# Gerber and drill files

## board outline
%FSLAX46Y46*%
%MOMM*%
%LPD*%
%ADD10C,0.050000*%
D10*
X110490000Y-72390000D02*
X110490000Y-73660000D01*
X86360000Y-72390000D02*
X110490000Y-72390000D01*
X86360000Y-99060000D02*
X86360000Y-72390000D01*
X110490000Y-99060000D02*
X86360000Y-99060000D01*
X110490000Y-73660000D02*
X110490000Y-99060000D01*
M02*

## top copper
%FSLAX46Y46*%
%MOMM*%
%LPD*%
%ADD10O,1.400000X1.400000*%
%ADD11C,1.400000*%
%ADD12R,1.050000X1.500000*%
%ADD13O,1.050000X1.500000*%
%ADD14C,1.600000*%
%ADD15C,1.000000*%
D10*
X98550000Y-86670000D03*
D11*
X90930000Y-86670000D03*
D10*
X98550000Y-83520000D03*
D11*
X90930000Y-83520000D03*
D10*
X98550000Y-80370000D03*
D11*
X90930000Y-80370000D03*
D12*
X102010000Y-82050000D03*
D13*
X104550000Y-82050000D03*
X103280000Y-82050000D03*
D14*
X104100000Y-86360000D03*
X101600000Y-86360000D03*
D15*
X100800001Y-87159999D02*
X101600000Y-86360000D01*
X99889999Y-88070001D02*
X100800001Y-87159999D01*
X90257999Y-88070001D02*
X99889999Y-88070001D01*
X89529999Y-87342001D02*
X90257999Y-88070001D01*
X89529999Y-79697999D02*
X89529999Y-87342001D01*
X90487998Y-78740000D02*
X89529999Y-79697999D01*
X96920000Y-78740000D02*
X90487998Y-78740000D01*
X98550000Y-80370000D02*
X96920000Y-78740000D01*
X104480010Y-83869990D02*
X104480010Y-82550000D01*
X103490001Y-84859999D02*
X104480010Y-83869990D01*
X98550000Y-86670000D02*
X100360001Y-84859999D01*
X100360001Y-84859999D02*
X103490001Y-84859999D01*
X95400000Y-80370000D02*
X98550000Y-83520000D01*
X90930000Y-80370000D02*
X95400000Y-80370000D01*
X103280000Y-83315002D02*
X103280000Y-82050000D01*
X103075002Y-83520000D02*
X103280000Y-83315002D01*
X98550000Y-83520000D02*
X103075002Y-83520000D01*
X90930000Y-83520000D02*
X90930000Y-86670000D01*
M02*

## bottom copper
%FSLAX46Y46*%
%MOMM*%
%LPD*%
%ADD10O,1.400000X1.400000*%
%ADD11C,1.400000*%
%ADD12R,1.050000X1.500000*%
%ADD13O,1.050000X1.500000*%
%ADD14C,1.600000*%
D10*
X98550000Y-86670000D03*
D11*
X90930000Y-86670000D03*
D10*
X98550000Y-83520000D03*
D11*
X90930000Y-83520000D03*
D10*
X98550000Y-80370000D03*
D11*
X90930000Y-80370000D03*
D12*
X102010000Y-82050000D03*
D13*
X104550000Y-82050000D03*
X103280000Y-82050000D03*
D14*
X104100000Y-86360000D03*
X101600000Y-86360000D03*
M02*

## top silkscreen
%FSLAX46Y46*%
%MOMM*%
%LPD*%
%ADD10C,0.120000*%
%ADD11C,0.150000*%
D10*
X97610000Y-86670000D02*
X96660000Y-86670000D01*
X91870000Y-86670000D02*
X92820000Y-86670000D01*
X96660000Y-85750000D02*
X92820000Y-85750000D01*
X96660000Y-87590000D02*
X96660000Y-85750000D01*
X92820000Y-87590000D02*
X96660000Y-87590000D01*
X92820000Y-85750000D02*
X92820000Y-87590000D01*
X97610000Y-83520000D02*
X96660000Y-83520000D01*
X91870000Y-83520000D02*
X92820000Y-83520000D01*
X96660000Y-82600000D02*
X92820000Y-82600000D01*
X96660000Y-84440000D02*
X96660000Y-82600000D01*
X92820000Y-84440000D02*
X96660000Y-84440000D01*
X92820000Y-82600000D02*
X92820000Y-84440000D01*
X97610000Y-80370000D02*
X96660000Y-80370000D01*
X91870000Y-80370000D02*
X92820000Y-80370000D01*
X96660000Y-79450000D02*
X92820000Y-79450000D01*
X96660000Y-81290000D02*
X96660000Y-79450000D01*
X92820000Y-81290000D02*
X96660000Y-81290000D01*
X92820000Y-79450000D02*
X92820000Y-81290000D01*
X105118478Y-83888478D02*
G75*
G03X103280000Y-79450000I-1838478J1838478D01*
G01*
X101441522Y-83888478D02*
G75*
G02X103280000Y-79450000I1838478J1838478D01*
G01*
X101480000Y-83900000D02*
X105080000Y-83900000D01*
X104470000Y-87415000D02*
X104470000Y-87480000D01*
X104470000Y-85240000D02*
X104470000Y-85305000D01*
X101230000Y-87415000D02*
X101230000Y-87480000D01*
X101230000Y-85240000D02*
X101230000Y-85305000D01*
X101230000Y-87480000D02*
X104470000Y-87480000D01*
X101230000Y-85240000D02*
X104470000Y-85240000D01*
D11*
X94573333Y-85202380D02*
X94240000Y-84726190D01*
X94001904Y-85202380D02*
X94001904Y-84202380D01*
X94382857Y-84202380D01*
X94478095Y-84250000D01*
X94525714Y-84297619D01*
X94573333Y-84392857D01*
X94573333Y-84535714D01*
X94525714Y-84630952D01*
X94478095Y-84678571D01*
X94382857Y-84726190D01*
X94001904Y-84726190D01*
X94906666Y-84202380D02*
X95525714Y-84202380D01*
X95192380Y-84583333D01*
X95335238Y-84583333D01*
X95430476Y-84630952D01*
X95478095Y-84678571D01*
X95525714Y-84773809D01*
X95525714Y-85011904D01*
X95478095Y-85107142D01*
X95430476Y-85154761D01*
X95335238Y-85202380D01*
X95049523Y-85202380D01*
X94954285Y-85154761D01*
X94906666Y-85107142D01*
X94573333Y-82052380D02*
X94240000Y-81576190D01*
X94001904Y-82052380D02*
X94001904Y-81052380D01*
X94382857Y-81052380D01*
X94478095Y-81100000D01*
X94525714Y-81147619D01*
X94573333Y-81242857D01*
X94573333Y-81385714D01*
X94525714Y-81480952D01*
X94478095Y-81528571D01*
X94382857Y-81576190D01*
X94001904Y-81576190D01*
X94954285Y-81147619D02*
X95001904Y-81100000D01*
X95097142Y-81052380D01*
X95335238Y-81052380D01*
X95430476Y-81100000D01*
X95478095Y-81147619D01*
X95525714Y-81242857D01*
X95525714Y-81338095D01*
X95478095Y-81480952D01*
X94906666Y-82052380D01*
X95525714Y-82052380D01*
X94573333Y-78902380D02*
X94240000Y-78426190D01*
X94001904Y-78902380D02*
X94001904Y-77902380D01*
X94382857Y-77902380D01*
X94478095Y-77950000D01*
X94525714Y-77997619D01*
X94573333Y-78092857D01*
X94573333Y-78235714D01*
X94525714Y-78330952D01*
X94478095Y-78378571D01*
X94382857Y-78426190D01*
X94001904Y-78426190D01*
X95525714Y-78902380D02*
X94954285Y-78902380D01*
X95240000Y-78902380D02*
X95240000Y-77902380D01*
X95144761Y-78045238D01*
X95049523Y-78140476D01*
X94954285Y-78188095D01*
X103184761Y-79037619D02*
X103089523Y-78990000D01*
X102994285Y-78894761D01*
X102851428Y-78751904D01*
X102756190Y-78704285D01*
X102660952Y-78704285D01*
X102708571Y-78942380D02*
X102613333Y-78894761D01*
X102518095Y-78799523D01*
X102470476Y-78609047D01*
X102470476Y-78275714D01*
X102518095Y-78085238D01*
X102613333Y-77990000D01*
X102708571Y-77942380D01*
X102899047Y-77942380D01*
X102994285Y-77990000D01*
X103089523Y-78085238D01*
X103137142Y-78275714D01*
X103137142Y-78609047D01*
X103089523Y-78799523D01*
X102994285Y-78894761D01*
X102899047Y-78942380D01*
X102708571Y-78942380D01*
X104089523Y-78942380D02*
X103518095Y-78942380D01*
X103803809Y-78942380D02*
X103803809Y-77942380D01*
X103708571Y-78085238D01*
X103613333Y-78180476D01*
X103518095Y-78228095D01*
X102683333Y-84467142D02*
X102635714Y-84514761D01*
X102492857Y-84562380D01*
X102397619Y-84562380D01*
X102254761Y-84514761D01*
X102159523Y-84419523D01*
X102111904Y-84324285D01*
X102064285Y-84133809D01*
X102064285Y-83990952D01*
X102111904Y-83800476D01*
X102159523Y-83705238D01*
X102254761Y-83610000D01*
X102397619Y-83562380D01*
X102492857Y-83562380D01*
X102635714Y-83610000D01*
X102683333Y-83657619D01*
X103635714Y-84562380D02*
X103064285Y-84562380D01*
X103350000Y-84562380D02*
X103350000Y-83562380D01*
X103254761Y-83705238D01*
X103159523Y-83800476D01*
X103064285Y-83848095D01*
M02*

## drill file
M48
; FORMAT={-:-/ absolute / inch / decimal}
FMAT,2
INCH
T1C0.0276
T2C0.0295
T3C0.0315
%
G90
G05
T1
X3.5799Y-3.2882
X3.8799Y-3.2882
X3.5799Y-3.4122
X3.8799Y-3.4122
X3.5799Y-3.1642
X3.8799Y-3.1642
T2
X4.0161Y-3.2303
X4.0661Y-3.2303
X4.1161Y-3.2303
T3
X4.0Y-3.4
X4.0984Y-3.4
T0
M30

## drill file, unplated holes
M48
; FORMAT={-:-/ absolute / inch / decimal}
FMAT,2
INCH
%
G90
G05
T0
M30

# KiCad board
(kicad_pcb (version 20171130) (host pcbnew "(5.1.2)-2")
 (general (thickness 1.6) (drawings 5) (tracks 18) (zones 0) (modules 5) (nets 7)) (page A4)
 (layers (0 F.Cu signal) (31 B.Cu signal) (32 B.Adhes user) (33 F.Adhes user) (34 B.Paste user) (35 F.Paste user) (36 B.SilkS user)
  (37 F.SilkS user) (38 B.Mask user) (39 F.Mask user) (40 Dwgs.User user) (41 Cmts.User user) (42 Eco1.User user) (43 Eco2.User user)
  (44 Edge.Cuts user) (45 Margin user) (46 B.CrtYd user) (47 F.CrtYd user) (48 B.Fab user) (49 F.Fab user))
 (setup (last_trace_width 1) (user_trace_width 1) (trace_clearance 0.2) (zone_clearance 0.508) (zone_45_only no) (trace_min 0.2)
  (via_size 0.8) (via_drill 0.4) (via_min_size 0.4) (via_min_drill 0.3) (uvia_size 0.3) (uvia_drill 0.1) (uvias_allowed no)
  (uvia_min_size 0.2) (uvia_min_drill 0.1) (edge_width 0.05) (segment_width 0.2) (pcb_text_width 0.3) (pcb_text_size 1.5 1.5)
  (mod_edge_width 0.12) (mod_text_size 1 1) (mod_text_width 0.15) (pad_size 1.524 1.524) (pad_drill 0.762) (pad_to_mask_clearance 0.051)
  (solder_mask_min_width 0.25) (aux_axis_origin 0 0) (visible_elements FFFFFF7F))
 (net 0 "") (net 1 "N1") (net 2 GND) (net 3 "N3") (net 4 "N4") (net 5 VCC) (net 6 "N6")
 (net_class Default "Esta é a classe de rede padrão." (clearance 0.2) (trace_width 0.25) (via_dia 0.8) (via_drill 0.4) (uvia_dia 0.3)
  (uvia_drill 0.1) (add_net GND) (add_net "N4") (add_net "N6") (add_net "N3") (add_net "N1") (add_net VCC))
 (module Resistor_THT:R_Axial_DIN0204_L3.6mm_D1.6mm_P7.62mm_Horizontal (layer F.Cu) (at 90.93 86.67)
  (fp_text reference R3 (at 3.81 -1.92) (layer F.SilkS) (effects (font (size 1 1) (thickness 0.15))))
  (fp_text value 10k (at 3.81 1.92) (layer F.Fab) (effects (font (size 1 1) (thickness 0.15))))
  (fp_line (start 6.68 0) (end 5.73 0) (layer F.SilkS) (width 0.12))
  (fp_line (start 0.94 0) (end 1.89 0) (layer F.SilkS) (width 0.12))
  (fp_line (start 5.73 -0.92) (end 1.89 -0.92) (layer F.SilkS) (width 0.12))
  (fp_line (start 5.73 0.92) (end 5.73 -0.92) (layer F.SilkS) (width 0.12))
  (fp_line (start 1.89 0.92) (end 5.73 0.92) (layer F.SilkS) (width 0.12))
  (fp_line (start 1.89 -0.92) (end 1.89 0.92) (layer F.SilkS) (width 0.12))
  (pad 2 thru_hole oval (at 7.62 0) (size 1.4 1.4) (drill 0.7) (layers *.Cu *.Mask) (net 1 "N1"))
  (pad 1 thru_hole circle (at 0 0) (size 1.4 1.4) (drill 0.7) (layers *.Cu *.Mask) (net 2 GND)))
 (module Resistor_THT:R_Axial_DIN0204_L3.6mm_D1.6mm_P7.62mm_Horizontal (layer F.Cu) (at 90.93 83.52)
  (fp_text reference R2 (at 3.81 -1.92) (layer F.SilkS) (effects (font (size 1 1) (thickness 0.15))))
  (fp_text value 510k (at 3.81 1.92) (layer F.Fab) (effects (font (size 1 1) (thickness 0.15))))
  (fp_line (start 6.68 0) (end 5.73 0) (layer F.SilkS) (width 0.12))
  (fp_line (start 0.94 0) (end 1.89 0) (layer F.SilkS) (width 0.12))
  (fp_line (start 5.73 -0.92) (end 1.89 -0.92) (layer F.SilkS) (width 0.12))
  (fp_line (start 5.73 0.92) (end 5.73 -0.92) (layer F.SilkS) (width 0.12))
  (fp_line (start 1.89 0.92) (end 5.73 0.92) (layer F.SilkS) (width 0.12))
  (fp_line (start 1.89 -0.92) (end 1.89 0.92) (layer F.SilkS) (width 0.12))
  (pad 2 thru_hole oval (at 7.62 0) (size 1.4 1.4) (drill 0.7) (layers *.Cu *.Mask) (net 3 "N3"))
  (pad 1 thru_hole circle (at 0 0) (size 1.4 1.4) (drill 0.7) (layers *.Cu *.Mask) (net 2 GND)))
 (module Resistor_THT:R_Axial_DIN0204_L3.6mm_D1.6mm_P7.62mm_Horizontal (layer F.Cu) (at 90.93 80.37)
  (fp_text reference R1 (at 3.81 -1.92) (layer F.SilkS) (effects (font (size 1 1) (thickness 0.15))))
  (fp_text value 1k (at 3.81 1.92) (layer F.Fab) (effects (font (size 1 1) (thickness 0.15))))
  (fp_line (start 6.68 0) (end 5.73 0) (layer F.SilkS) (width 0.12))
  (fp_line (start 0.94 0) (end 1.89 0) (layer F.SilkS) (width 0.12))
  (fp_line (start 5.73 -0.92) (end 1.89 -0.92) (layer F.SilkS) (width 0.12))
  (fp_line (start 5.73 0.92) (end 5.73 -0.92) (layer F.SilkS) (width 0.12))
  (fp_line (start 1.89 0.92) (end 5.73 0.92) (layer F.SilkS) (width 0.12))
  (fp_line (start 1.89 -0.92) (end 1.89 0.92) (layer F.SilkS) (width 0.12))
  (pad 2 thru_hole oval (at 7.62 0) (size 1.4 1.4) (drill 0.7) (layers *.Cu *.Mask) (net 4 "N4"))
  (pad 1 thru_hole circle (at 0 0) (size 1.4 1.4) (drill 0.7) (layers *.Cu *.Mask) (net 3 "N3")))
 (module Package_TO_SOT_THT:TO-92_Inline (layer F.Cu) (at 102.01 82.05)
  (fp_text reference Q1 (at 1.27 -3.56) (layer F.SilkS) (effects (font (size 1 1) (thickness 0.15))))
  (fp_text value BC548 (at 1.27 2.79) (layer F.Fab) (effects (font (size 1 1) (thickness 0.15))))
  (fp_arc (start 1.27 0) (end 1.27 -2.6) (angle 135) (layer F.SilkS) (width 0.12))
  (fp_arc (start 1.27 0) (end 1.27 -2.6) (angle -135) (layer F.SilkS) (width 0.12))
  (fp_line (start -0.53 1.85) (end 3.07 1.85) (layer F.SilkS) (width 0.12))
  (pad 1 thru_hole rect (at 0 0) (size 1.05 1.5) (drill 0.75) (layers *.Cu *.Mask) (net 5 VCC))
  (pad 3 thru_hole oval (at 2.54 0) (size 1.05 1.5) (drill 0.75) (layers *.Cu *.Mask) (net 1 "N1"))
  (pad 2 thru_hole oval (at 1.27 0) (size 1.05 1.5) (drill 0.75) (layers *.Cu *.Mask) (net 3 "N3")))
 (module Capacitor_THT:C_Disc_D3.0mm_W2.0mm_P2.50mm (layer F.Cu) (at 101.6 86.36)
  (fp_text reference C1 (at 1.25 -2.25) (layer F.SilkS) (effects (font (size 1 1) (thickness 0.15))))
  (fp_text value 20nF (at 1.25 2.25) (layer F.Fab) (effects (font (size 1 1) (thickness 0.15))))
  (fp_line (start 2.87 1.055) (end 2.87 1.12) (layer F.SilkS) (width 0.12))
  (fp_line (start 2.87 -1.12) (end 2.87 -1.055) (layer F.SilkS) (width 0.12))
  (fp_line (start -0.37 1.055) (end -0.37 1.12) (layer F.SilkS) (width 0.12))
  (fp_line (start -0.37 -1.12) (end -0.37 -1.055) (layer F.SilkS) (width 0.12))
  (fp_line (start -0.37 1.12) (end 2.87 1.12) (layer F.SilkS) (width 0.12))
  (fp_line (start -0.37 -1.12) (end 2.87 -1.12) (layer F.SilkS) (width 0.12))
  (pad 2 thru_hole circle (at 2.5 0) (size 1.6 1.6) (drill 0.8) (layers *.Cu *.Mask) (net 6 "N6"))
  (pad 1 thru_hole circle (at 0 0) (size 1.6 1.6) (drill 0.8) (layers *.Cu *.Mask) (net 4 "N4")))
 (gr_line (start 110.49 72.39) (end 110.49 73.66) (layer Edge.Cuts) (width 0.05))
 (gr_line (start 86.36 72.39) (end 110.49 72.39) (layer Edge.Cuts) (width 0.05))
 (gr_line (start 86.36 99.06) (end 86.36 72.39) (layer Edge.Cuts) (width 0.05))
 (gr_line (start 110.49 99.06) (end 86.36 99.06) (layer Edge.Cuts) (width 0.05))
 (gr_line (start 110.49 73.66) (end 110.49 99.06) (layer Edge.Cuts) (width 0.05))
 (segment (start 100.800001 87.159999) (end 101.6 86.36) (width 1) (layer F.Cu) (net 4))
 (segment (start 99.889999 88.070001) (end 100.800001 87.159999) (width 1) (layer F.Cu) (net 4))
 (segment (start 90.257999 88.070001) (end 99.889999 88.070001) (width 1) (layer F.Cu) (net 4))
 (segment (start 89.529999 87.342001) (end 90.257999 88.070001) (width 1) (layer F.Cu) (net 4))
 (segment (start 89.529999 79.697999) (end 89.529999 87.342001) (width 1) (layer F.Cu) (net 4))
 (segment (start 90.487998 78.74) (end 89.529999 79.697999) (width 1) (layer F.Cu) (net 4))
 (segment (start 96.92 78.74) (end 90.487998 78.74) (width 1) (layer F.Cu) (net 4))
 (segment (start 98.55 80.37) (end 96.92 78.74) (width 1) (layer F.Cu) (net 4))
 (segment (start 104.48001 83.86999) (end 104.48001 82.55) (width 1) (layer F.Cu) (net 1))
 (segment (start 103.490001 84.859999) (end 104.48001 83.86999) (width 1) (layer F.Cu) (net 1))
 (segment (start 98.55 86.67) (end 100.360001 84.859999) (width 1) (layer F.Cu) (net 1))
 (segment (start 100.360001 84.859999) (end 103.490001 84.859999) (width 1) (layer F.Cu) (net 1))
 (segment (start 95.4 80.37) (end 98.55 83.52) (width 1) (layer F.Cu) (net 3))
 (segment (start 90.93 80.37) (end 95.4 80.37) (width 1) (layer F.Cu) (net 3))
 (segment (start 103.28 83.315002) (end 103.28 82.05) (width 1) (layer F.Cu) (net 3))
 (segment (start 103.075002 83.52) (end 103.28 83.315002) (width 1) (layer F.Cu) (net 3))
 (segment (start 98.55 83.52) (end 103.075002 83.52) (width 1) (layer F.Cu) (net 3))
 (segment (start 90.93 83.52) (end 90.93 86.67) (width 1) (layer F.Cu) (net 2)))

